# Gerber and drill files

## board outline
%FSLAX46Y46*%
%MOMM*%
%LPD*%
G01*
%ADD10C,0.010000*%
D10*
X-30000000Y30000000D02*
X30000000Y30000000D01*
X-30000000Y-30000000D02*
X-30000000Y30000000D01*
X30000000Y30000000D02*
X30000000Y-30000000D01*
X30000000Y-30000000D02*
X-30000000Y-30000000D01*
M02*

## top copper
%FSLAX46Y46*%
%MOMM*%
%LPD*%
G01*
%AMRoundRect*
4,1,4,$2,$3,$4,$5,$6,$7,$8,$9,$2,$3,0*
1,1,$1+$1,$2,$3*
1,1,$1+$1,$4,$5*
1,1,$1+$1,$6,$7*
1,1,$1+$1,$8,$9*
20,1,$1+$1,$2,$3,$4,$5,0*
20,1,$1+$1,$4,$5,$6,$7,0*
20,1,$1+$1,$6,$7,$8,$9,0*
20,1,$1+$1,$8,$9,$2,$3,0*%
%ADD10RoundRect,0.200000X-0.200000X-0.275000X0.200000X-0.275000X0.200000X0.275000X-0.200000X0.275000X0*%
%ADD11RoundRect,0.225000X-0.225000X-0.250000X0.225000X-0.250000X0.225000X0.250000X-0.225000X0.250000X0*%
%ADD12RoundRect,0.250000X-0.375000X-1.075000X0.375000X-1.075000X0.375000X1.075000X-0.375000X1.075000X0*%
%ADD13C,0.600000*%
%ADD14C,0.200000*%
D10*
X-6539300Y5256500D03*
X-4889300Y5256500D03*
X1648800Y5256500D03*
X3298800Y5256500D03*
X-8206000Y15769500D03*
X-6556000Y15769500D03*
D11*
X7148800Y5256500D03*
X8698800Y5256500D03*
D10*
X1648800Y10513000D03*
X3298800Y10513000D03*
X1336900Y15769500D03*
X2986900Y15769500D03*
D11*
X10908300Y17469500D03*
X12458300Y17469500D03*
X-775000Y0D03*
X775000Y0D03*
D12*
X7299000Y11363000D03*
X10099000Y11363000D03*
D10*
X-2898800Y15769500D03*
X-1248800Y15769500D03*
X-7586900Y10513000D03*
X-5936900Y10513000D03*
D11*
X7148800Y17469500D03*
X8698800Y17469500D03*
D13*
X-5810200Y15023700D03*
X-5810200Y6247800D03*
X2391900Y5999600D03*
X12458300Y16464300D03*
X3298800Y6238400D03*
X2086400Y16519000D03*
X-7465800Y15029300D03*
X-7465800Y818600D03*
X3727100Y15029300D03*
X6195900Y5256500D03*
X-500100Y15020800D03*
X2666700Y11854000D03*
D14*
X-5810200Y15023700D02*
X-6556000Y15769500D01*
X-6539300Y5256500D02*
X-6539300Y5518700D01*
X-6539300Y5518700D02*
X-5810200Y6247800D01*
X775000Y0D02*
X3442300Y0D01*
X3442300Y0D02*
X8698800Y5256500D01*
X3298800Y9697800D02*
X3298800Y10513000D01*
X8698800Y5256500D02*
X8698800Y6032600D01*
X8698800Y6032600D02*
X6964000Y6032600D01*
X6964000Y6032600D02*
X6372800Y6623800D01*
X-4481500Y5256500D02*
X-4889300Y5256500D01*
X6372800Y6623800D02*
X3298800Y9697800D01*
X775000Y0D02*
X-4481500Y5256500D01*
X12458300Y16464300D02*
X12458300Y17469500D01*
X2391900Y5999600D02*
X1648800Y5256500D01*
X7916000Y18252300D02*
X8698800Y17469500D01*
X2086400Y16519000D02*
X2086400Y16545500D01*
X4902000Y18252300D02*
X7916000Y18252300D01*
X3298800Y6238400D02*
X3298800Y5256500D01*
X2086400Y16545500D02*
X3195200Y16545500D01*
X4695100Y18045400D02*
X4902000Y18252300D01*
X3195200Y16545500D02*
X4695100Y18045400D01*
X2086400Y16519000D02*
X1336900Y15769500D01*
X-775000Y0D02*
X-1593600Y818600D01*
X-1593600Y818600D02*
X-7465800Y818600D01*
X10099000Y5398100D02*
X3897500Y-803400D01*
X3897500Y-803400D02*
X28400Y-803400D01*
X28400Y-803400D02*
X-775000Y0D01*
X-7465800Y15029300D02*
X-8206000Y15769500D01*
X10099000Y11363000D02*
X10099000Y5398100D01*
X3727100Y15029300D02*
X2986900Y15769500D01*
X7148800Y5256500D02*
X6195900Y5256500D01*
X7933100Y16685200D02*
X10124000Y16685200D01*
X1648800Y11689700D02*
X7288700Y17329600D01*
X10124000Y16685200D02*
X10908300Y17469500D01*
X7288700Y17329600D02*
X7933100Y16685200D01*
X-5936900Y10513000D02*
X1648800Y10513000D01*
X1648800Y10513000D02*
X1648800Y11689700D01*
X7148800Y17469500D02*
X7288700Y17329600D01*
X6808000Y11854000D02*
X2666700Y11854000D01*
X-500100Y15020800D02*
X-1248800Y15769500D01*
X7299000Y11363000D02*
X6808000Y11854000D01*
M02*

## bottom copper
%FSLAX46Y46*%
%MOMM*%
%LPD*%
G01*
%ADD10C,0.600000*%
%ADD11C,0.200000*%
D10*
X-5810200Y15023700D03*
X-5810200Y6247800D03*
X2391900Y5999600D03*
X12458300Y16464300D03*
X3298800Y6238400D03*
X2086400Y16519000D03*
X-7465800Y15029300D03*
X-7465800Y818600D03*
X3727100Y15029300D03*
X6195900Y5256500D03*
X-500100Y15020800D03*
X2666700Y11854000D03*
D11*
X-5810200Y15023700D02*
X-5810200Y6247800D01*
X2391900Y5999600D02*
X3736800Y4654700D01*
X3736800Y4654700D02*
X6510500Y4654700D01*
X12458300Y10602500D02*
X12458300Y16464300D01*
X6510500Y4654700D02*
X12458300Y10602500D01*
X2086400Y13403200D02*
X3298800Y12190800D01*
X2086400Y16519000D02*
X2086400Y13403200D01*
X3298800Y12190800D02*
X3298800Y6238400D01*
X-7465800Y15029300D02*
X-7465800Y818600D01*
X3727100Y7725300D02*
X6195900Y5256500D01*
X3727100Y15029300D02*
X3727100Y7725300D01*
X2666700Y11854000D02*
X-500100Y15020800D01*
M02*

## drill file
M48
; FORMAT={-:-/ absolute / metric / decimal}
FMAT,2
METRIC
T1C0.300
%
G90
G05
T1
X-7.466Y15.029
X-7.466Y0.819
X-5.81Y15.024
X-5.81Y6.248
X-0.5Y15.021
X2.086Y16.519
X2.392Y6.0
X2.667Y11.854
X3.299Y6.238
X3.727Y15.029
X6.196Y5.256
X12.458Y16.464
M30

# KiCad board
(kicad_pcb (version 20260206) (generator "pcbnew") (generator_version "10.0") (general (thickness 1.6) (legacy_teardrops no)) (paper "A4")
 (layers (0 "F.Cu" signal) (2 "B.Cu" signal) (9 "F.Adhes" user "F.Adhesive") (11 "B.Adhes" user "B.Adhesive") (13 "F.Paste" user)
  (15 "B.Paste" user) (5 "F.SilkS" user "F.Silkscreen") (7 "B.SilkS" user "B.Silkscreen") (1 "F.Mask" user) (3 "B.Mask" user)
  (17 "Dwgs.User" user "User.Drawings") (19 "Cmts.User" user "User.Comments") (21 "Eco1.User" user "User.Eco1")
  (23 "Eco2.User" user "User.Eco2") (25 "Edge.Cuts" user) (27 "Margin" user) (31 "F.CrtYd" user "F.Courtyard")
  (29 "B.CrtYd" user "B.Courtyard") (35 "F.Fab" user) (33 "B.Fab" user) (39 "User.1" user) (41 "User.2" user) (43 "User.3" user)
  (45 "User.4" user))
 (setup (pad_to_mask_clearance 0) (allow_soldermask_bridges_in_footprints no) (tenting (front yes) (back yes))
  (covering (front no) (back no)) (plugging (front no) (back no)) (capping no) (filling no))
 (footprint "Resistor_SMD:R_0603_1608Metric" (layer "F.Cu") (at -5.7143 -5.2565)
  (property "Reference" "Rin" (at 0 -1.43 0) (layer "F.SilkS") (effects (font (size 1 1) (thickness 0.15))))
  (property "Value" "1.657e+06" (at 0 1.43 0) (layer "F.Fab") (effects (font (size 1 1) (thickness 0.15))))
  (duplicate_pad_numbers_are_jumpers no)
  (pad "1" smd roundrect (at -0.825 0) (size 0.8 0.95) (layers "F.Cu" "F.Mask" "F.Paste") (roundrect_rratio 0.25) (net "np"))
  (pad "2" smd roundrect (at 0.825 0) (size 0.8 0.95) (layers "F.Cu" "F.Mask" "F.Paste") (roundrect_rratio 0.25) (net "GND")))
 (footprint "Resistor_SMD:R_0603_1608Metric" (layer "F.Cu") (at 2.4738 -5.2565)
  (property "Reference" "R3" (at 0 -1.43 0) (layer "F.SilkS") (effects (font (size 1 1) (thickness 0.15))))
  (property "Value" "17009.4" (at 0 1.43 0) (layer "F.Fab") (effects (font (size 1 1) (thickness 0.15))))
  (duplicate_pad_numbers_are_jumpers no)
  (pad "1" smd roundrect (at -0.825 0) (size 0.8 0.95) (layers "F.Cu" "F.Mask" "F.Paste") (roundrect_rratio 0.25) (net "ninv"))
  (pad "2" smd roundrect (at 0.825 0) (size 0.8 0.95) (layers "F.Cu" "F.Mask" "F.Paste") (roundrect_rratio 0.25) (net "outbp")))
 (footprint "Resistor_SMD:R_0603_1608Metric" (layer "F.Cu") (at -7.381 -15.7695)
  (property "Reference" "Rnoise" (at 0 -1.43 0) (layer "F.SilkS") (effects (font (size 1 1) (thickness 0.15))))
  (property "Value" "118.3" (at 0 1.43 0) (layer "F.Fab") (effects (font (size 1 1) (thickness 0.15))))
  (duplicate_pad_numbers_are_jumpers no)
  (pad "1" smd roundrect (at -0.825 0) (size 0.8 0.95) (layers "F.Cu" "F.Mask" "F.Paste") (roundrect_rratio 0.25) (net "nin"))
  (pad "2" smd roundrect (at 0.825 0) (size 0.8 0.95) (layers "F.Cu" "F.Mask" "F.Paste") (roundrect_rratio 0.25) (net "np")))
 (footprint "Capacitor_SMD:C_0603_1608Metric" (layer "F.Cu") (at 7.9238 -5.2565)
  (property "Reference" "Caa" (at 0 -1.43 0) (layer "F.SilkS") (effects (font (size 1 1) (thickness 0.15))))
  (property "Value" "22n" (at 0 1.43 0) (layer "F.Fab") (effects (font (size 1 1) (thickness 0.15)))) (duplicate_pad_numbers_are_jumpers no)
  (pad "1" smd roundrect (at -0.775 0) (size 0.9 0.95) (layers "F.Cu" "F.Mask" "F.Paste") (roundrect_rratio 0.25) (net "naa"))
  (pad "2" smd roundrect (at 0.775 0) (size 0.9 0.95) (layers "F.Cu" "F.Mask" "F.Paste") (roundrect_rratio 0.25) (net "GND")))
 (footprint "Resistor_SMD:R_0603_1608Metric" (layer "F.Cu") (at 2.4738 -10.513)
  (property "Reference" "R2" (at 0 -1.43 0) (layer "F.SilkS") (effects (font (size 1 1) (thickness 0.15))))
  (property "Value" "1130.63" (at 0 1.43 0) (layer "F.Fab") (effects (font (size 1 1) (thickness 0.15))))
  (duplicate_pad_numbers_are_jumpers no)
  (pad "1" smd roundrect (at -0.825 0) (size 0.8 0.95) (layers "F.Cu" "F.Mask" "F.Paste") (roundrect_rratio 0.25) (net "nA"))
  (pad "2" smd roundrect (at 0.825 0) (size 0.8 0.95) (layers "F.Cu" "F.Mask" "F.Paste") (roundrect_rratio 0.25) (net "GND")))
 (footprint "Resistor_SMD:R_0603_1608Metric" (layer "F.Cu") (at 2.1619 -15.7695)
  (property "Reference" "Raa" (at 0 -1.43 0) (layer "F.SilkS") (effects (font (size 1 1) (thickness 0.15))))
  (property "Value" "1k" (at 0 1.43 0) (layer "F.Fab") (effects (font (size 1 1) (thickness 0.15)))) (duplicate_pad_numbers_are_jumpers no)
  (pad "1" smd roundrect (at -0.825 0) (size 0.8 0.95) (layers "F.Cu" "F.Mask" "F.Paste") (roundrect_rratio 0.25) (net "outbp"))
  (pad "2" smd roundrect (at 0.825 0) (size 0.8 0.95) (layers "F.Cu" "F.Mask" "F.Paste") (roundrect_rratio 0.25) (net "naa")))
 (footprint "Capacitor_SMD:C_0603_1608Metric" (layer "F.Cu") (at 11.6833 -17.4695)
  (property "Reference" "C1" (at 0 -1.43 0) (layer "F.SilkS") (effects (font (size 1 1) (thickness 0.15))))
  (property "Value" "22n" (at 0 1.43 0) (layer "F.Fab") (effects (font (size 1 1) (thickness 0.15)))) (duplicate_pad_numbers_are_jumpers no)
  (pad "1" smd roundrect (at -0.775 0) (size 0.9 0.95) (layers "F.Cu" "F.Mask" "F.Paste") (roundrect_rratio 0.25) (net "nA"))
  (pad "2" smd roundrect (at 0.775 0) (size 0.9 0.95) (layers "F.Cu" "F.Mask" "F.Paste") (roundrect_rratio 0.25) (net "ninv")))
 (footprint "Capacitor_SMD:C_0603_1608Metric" (layer "F.Cu") (at 0 0)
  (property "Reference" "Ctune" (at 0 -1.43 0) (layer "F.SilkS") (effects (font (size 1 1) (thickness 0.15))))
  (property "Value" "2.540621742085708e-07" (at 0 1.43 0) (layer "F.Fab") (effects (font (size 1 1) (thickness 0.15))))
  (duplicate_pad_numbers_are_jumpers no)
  (pad "1" smd roundrect (at -0.775 0) (size 0.9 0.95) (layers "F.Cu" "F.Mask" "F.Paste") (roundrect_rratio 0.25) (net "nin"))
  (pad "2" smd roundrect (at 0.775 0) (size 0.9 0.95) (layers "F.Cu" "F.Mask" "F.Paste") (roundrect_rratio 0.25) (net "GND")))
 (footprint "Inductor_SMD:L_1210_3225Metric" (layer "F.Cu") (at 8.699 -11.363)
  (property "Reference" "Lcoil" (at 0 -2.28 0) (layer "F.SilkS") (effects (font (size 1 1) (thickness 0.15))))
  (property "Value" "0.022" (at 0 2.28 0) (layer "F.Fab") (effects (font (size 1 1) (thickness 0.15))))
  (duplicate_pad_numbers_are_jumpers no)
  (pad "1" smd roundrect (at -1.4 0) (size 1.25 2.65) (layers "F.Cu" "F.Mask" "F.Paste") (roundrect_rratio 0.2) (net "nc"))
  (pad "2" smd roundrect (at 1.4 0) (size 1.25 2.65) (layers "F.Cu" "F.Mask" "F.Paste") (roundrect_rratio 0.2) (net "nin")))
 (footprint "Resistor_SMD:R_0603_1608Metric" (layer "F.Cu") (at -2.0738 -15.7695)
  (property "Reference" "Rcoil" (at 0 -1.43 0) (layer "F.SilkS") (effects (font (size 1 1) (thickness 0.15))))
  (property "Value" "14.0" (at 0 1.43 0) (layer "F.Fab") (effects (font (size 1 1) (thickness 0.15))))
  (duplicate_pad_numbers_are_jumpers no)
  (pad "1" smd roundrect (at -0.825 0) (size 0.8 0.95) (layers "F.Cu" "F.Mask" "F.Paste") (roundrect_rratio 0.25) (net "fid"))
  (pad "2" smd roundrect (at 0.825 0) (size 0.8 0.95) (layers "F.Cu" "F.Mask" "F.Paste") (roundrect_rratio 0.25) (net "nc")))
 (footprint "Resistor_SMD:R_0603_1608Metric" (layer "F.Cu") (at -6.7619 -10.513)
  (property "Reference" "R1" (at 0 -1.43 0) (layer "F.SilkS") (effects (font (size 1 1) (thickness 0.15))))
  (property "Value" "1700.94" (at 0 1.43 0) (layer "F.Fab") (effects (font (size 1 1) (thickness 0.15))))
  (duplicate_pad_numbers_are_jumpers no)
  (pad "1" smd roundrect (at -0.825 0) (size 0.8 0.95) (layers "F.Cu" "F.Mask" "F.Paste") (roundrect_rratio 0.25) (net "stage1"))
  (pad "2" smd roundrect (at 0.825 0) (size 0.8 0.95) (layers "F.Cu" "F.Mask" "F.Paste") (roundrect_rratio 0.25) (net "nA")))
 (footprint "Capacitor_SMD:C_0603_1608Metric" (layer "F.Cu") (at 7.9238 -17.4695)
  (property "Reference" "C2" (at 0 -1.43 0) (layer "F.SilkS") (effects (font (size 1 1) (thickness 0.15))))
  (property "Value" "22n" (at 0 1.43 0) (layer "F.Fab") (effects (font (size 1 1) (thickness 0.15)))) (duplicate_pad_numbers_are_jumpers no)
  (pad "1" smd roundrect (at -0.775 0) (size 0.9 0.95) (layers "F.Cu" "F.Mask" "F.Paste") (roundrect_rratio 0.25) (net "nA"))
  (pad "2" smd roundrect (at 0.775 0) (size 0.9 0.95) (layers "F.Cu" "F.Mask" "F.Paste") (roundrect_rratio 0.25) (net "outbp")))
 (gr_line (start -30 -30) (end 30 -30) (stroke (width 0.01) (type default)) (layer "Edge.Cuts"))
 (gr_line (start -30 30) (end -30 -30) (stroke (width 0.01) (type default)) (layer "Edge.Cuts"))
 (gr_line (start 30 -30) (end 30 30) (stroke (width 0.01) (type default)) (layer "Edge.Cuts"))
 (gr_line (start 30 30) (end -30 30) (stroke (width 0.01) (type default)) (layer "Edge.Cuts"))
 (segment (start -5.8102 -15.0237) (end -6.556 -15.7695) (width 0.2) (layer "F.Cu") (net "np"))
 (segment (start -6.5393 -5.2565) (end -6.5393 -5.5187) (width 0.2) (layer "F.Cu") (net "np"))
 (segment (start -6.5393 -5.5187) (end -5.8102 -6.2478) (width 0.2) (layer "F.Cu") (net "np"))
 (via (at -5.8102 -15.0237) (size 0.6) (drill 0.3) (layers "F.Cu" "B.Cu") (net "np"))
 (via (at -5.8102 -6.2478) (size 0.6) (drill 0.3) (layers "F.Cu" "B.Cu") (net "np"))
 (segment (start -5.8102 -15.0237) (end -5.8102 -6.2478) (width 0.2) (layer "B.Cu") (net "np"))
 (segment (start 0.775 0) (end 3.4423 0) (width 0.2) (layer "F.Cu") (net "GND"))
 (segment (start 3.4423 0) (end 8.6988 -5.2565) (width 0.2) (layer "F.Cu") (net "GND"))
 (segment (start 3.2988 -9.6978) (end 3.2988 -10.513) (width 0.2) (layer "F.Cu") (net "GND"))
 (segment (start 8.6988 -5.2565) (end 8.6988 -6.0326) (width 0.2) (layer "F.Cu") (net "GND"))
 (segment (start 8.6988 -6.0326) (end 6.964 -6.0326) (width 0.2) (layer "F.Cu") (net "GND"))
 (segment (start 6.964 -6.0326) (end 6.3728 -6.6238) (width 0.2) (layer "F.Cu") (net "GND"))
 (segment (start -4.4815 -5.2565) (end -4.8893 -5.2565) (width 0.2) (layer "F.Cu") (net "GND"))
 (segment (start 6.3728 -6.6238) (end 3.2988 -9.6978) (width 0.2) (layer "F.Cu") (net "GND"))
 (segment (start 0.775 0) (end -4.4815 -5.2565) (width 0.2) (layer "F.Cu") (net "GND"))
 (segment (start 12.4583 -16.4643) (end 12.4583 -17.4695) (width 0.2) (layer "F.Cu") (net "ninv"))
 (segment (start 2.3919 -5.9996) (end 1.6488 -5.2565) (width 0.2) (layer "F.Cu") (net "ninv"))
 (via (at 2.3919 -5.9996) (size 0.6) (drill 0.3) (layers "F.Cu" "B.Cu") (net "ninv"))
 (via (at 12.4583 -16.4643) (size 0.6) (drill 0.3) (layers "F.Cu" "B.Cu") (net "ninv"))
 (segment (start 2.3919 -5.9996) (end 3.7368 -4.6547) (width 0.2) (layer "B.Cu") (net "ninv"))
 (segment (start 3.7368 -4.6547) (end 6.5105 -4.6547) (width 0.2) (layer "B.Cu") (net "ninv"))
 (segment (start 12.4583 -10.6025) (end 12.4583 -16.4643) (width 0.2) (layer "B.Cu") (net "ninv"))
 (segment (start 6.5105 -4.6547) (end 12.4583 -10.6025) (width 0.2) (layer "B.Cu") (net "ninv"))
 (segment (start 7.916 -18.2523) (end 8.6988 -17.4695) (width 0.2) (layer "F.Cu") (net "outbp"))
 (segment (start 2.0864 -16.519) (end 2.0864 -16.5455) (width 0.2) (layer "F.Cu") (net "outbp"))
 (segment (start 4.902 -18.2523) (end 7.916 -18.2523) (width 0.2) (layer "F.Cu") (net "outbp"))
 (segment (start 3.2988 -6.2384) (end 3.2988 -5.2565) (width 0.2) (layer "F.Cu") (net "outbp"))
 (segment (start 2.0864 -16.5455) (end 3.1952 -16.5455) (width 0.2) (layer "F.Cu") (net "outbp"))
 (segment (start 4.6951 -18.0454) (end 4.902 -18.2523) (width 0.2) (layer "F.Cu") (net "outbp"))
 (segment (start 3.1952 -16.5455) (end 4.6951 -18.0454) (width 0.2) (layer "F.Cu") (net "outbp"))
 (segment (start 2.0864 -16.519) (end 1.3369 -15.7695) (width 0.2) (layer "F.Cu") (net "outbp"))
 (via (at 3.2988 -6.2384) (size 0.6) (drill 0.3) (layers "F.Cu" "B.Cu") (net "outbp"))
 (via (at 2.0864 -16.519) (size 0.6) (drill 0.3) (layers "F.Cu" "B.Cu") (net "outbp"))
 (segment (start 2.0864 -13.4032) (end 3.2988 -12.1908) (width 0.2) (layer "B.Cu") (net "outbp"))
 (segment (start 2.0864 -16.519) (end 2.0864 -13.4032) (width 0.2) (layer "B.Cu") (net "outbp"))
 (segment (start 3.2988 -12.1908) (end 3.2988 -6.2384) (width 0.2) (layer "B.Cu") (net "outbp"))
 (segment (start -0.775 0) (end -1.5936 -0.8186) (width 0.2) (layer "F.Cu") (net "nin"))
 (segment (start -1.5936 -0.8186) (end -7.4658 -0.8186) (width 0.2) (layer "F.Cu") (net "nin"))
 (segment (start 10.099 -5.3981) (end 3.8975 0.8034) (width 0.2) (layer "F.Cu") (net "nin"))
 (segment (start 3.8975 0.8034) (end 0.0284 0.8034) (width 0.2) (layer "F.Cu") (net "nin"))
 (segment (start 0.0284 0.8034) (end -0.775 0) (width 0.2) (layer "F.Cu") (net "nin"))
 (segment (start -7.4658 -15.0293) (end -8.206 -15.7695) (width 0.2) (layer "F.Cu") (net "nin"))
 (segment (start 10.099 -11.363) (end 10.099 -5.3981) (width 0.2) (layer "F.Cu") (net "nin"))
 (via (at -7.4658 -15.0293) (size 0.6) (drill 0.3) (layers "F.Cu" "B.Cu") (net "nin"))
 (via (at -7.4658 -0.8186) (size 0.6) (drill 0.3) (layers "F.Cu" "B.Cu") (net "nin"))
 (segment (start -7.4658 -15.0293) (end -7.4658 -0.8186) (width 0.2) (layer "B.Cu") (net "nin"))
 (segment (start 3.7271 -15.0293) (end 2.9869 -15.7695) (width 0.2) (layer "F.Cu") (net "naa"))
 (segment (start 7.1488 -5.2565) (end 6.1959 -5.2565) (width 0.2) (layer "F.Cu") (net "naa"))
 (via (at 3.7271 -15.0293) (size 0.6) (drill 0.3) (layers "F.Cu" "B.Cu") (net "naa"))
 (via (at 6.1959 -5.2565) (size 0.6) (drill 0.3) (layers "F.Cu" "B.Cu") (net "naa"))
 (segment (start 3.7271 -7.7253) (end 6.1959 -5.2565) (width 0.2) (layer "B.Cu") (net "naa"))
 (segment (start 3.7271 -15.0293) (end 3.7271 -7.7253) (width 0.2) (layer "B.Cu") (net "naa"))
 (segment (start 7.9331 -16.6852) (end 10.124 -16.6852) (width 0.2) (layer "F.Cu") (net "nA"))
 (segment (start 1.6488 -11.6897) (end 7.2887 -17.3296) (width 0.2) (layer "F.Cu") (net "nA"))
 (segment (start 10.124 -16.6852) (end 10.9083 -17.4695) (width 0.2) (layer "F.Cu") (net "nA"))
 (segment (start 7.2887 -17.3296) (end 7.9331 -16.6852) (width 0.2) (layer "F.Cu") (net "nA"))
 (segment (start -5.9369 -10.513) (end 1.6488 -10.513) (width 0.2) (layer "F.Cu") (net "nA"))
 (segment (start 1.6488 -10.513) (end 1.6488 -11.6897) (width 0.2) (layer "F.Cu") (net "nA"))
 (segment (start 7.1488 -17.4695) (end 7.2887 -17.3296) (width 0.2) (layer "F.Cu") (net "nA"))
 (segment (start 6.808 -11.854) (end 2.6667 -11.854) (width 0.2) (layer "F.Cu") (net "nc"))
 (segment (start -0.5001 -15.0208) (end -1.2488 -15.7695) (width 0.2) (layer "F.Cu") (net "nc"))
 (segment (start 7.299 -11.363) (end 6.808 -11.854) (width 0.2) (layer "F.Cu") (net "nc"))
 (via (at -0.5001 -15.0208) (size 0.6) (drill 0.3) (layers "F.Cu" "B.Cu") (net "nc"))
 (via (at 2.6667 -11.854) (size 0.6) (drill 0.3) (layers "F.Cu" "B.Cu") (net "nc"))
 (segment (start 2.6667 -11.854) (end -0.5001 -15.0208) (width 0.2) (layer "B.Cu") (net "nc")))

